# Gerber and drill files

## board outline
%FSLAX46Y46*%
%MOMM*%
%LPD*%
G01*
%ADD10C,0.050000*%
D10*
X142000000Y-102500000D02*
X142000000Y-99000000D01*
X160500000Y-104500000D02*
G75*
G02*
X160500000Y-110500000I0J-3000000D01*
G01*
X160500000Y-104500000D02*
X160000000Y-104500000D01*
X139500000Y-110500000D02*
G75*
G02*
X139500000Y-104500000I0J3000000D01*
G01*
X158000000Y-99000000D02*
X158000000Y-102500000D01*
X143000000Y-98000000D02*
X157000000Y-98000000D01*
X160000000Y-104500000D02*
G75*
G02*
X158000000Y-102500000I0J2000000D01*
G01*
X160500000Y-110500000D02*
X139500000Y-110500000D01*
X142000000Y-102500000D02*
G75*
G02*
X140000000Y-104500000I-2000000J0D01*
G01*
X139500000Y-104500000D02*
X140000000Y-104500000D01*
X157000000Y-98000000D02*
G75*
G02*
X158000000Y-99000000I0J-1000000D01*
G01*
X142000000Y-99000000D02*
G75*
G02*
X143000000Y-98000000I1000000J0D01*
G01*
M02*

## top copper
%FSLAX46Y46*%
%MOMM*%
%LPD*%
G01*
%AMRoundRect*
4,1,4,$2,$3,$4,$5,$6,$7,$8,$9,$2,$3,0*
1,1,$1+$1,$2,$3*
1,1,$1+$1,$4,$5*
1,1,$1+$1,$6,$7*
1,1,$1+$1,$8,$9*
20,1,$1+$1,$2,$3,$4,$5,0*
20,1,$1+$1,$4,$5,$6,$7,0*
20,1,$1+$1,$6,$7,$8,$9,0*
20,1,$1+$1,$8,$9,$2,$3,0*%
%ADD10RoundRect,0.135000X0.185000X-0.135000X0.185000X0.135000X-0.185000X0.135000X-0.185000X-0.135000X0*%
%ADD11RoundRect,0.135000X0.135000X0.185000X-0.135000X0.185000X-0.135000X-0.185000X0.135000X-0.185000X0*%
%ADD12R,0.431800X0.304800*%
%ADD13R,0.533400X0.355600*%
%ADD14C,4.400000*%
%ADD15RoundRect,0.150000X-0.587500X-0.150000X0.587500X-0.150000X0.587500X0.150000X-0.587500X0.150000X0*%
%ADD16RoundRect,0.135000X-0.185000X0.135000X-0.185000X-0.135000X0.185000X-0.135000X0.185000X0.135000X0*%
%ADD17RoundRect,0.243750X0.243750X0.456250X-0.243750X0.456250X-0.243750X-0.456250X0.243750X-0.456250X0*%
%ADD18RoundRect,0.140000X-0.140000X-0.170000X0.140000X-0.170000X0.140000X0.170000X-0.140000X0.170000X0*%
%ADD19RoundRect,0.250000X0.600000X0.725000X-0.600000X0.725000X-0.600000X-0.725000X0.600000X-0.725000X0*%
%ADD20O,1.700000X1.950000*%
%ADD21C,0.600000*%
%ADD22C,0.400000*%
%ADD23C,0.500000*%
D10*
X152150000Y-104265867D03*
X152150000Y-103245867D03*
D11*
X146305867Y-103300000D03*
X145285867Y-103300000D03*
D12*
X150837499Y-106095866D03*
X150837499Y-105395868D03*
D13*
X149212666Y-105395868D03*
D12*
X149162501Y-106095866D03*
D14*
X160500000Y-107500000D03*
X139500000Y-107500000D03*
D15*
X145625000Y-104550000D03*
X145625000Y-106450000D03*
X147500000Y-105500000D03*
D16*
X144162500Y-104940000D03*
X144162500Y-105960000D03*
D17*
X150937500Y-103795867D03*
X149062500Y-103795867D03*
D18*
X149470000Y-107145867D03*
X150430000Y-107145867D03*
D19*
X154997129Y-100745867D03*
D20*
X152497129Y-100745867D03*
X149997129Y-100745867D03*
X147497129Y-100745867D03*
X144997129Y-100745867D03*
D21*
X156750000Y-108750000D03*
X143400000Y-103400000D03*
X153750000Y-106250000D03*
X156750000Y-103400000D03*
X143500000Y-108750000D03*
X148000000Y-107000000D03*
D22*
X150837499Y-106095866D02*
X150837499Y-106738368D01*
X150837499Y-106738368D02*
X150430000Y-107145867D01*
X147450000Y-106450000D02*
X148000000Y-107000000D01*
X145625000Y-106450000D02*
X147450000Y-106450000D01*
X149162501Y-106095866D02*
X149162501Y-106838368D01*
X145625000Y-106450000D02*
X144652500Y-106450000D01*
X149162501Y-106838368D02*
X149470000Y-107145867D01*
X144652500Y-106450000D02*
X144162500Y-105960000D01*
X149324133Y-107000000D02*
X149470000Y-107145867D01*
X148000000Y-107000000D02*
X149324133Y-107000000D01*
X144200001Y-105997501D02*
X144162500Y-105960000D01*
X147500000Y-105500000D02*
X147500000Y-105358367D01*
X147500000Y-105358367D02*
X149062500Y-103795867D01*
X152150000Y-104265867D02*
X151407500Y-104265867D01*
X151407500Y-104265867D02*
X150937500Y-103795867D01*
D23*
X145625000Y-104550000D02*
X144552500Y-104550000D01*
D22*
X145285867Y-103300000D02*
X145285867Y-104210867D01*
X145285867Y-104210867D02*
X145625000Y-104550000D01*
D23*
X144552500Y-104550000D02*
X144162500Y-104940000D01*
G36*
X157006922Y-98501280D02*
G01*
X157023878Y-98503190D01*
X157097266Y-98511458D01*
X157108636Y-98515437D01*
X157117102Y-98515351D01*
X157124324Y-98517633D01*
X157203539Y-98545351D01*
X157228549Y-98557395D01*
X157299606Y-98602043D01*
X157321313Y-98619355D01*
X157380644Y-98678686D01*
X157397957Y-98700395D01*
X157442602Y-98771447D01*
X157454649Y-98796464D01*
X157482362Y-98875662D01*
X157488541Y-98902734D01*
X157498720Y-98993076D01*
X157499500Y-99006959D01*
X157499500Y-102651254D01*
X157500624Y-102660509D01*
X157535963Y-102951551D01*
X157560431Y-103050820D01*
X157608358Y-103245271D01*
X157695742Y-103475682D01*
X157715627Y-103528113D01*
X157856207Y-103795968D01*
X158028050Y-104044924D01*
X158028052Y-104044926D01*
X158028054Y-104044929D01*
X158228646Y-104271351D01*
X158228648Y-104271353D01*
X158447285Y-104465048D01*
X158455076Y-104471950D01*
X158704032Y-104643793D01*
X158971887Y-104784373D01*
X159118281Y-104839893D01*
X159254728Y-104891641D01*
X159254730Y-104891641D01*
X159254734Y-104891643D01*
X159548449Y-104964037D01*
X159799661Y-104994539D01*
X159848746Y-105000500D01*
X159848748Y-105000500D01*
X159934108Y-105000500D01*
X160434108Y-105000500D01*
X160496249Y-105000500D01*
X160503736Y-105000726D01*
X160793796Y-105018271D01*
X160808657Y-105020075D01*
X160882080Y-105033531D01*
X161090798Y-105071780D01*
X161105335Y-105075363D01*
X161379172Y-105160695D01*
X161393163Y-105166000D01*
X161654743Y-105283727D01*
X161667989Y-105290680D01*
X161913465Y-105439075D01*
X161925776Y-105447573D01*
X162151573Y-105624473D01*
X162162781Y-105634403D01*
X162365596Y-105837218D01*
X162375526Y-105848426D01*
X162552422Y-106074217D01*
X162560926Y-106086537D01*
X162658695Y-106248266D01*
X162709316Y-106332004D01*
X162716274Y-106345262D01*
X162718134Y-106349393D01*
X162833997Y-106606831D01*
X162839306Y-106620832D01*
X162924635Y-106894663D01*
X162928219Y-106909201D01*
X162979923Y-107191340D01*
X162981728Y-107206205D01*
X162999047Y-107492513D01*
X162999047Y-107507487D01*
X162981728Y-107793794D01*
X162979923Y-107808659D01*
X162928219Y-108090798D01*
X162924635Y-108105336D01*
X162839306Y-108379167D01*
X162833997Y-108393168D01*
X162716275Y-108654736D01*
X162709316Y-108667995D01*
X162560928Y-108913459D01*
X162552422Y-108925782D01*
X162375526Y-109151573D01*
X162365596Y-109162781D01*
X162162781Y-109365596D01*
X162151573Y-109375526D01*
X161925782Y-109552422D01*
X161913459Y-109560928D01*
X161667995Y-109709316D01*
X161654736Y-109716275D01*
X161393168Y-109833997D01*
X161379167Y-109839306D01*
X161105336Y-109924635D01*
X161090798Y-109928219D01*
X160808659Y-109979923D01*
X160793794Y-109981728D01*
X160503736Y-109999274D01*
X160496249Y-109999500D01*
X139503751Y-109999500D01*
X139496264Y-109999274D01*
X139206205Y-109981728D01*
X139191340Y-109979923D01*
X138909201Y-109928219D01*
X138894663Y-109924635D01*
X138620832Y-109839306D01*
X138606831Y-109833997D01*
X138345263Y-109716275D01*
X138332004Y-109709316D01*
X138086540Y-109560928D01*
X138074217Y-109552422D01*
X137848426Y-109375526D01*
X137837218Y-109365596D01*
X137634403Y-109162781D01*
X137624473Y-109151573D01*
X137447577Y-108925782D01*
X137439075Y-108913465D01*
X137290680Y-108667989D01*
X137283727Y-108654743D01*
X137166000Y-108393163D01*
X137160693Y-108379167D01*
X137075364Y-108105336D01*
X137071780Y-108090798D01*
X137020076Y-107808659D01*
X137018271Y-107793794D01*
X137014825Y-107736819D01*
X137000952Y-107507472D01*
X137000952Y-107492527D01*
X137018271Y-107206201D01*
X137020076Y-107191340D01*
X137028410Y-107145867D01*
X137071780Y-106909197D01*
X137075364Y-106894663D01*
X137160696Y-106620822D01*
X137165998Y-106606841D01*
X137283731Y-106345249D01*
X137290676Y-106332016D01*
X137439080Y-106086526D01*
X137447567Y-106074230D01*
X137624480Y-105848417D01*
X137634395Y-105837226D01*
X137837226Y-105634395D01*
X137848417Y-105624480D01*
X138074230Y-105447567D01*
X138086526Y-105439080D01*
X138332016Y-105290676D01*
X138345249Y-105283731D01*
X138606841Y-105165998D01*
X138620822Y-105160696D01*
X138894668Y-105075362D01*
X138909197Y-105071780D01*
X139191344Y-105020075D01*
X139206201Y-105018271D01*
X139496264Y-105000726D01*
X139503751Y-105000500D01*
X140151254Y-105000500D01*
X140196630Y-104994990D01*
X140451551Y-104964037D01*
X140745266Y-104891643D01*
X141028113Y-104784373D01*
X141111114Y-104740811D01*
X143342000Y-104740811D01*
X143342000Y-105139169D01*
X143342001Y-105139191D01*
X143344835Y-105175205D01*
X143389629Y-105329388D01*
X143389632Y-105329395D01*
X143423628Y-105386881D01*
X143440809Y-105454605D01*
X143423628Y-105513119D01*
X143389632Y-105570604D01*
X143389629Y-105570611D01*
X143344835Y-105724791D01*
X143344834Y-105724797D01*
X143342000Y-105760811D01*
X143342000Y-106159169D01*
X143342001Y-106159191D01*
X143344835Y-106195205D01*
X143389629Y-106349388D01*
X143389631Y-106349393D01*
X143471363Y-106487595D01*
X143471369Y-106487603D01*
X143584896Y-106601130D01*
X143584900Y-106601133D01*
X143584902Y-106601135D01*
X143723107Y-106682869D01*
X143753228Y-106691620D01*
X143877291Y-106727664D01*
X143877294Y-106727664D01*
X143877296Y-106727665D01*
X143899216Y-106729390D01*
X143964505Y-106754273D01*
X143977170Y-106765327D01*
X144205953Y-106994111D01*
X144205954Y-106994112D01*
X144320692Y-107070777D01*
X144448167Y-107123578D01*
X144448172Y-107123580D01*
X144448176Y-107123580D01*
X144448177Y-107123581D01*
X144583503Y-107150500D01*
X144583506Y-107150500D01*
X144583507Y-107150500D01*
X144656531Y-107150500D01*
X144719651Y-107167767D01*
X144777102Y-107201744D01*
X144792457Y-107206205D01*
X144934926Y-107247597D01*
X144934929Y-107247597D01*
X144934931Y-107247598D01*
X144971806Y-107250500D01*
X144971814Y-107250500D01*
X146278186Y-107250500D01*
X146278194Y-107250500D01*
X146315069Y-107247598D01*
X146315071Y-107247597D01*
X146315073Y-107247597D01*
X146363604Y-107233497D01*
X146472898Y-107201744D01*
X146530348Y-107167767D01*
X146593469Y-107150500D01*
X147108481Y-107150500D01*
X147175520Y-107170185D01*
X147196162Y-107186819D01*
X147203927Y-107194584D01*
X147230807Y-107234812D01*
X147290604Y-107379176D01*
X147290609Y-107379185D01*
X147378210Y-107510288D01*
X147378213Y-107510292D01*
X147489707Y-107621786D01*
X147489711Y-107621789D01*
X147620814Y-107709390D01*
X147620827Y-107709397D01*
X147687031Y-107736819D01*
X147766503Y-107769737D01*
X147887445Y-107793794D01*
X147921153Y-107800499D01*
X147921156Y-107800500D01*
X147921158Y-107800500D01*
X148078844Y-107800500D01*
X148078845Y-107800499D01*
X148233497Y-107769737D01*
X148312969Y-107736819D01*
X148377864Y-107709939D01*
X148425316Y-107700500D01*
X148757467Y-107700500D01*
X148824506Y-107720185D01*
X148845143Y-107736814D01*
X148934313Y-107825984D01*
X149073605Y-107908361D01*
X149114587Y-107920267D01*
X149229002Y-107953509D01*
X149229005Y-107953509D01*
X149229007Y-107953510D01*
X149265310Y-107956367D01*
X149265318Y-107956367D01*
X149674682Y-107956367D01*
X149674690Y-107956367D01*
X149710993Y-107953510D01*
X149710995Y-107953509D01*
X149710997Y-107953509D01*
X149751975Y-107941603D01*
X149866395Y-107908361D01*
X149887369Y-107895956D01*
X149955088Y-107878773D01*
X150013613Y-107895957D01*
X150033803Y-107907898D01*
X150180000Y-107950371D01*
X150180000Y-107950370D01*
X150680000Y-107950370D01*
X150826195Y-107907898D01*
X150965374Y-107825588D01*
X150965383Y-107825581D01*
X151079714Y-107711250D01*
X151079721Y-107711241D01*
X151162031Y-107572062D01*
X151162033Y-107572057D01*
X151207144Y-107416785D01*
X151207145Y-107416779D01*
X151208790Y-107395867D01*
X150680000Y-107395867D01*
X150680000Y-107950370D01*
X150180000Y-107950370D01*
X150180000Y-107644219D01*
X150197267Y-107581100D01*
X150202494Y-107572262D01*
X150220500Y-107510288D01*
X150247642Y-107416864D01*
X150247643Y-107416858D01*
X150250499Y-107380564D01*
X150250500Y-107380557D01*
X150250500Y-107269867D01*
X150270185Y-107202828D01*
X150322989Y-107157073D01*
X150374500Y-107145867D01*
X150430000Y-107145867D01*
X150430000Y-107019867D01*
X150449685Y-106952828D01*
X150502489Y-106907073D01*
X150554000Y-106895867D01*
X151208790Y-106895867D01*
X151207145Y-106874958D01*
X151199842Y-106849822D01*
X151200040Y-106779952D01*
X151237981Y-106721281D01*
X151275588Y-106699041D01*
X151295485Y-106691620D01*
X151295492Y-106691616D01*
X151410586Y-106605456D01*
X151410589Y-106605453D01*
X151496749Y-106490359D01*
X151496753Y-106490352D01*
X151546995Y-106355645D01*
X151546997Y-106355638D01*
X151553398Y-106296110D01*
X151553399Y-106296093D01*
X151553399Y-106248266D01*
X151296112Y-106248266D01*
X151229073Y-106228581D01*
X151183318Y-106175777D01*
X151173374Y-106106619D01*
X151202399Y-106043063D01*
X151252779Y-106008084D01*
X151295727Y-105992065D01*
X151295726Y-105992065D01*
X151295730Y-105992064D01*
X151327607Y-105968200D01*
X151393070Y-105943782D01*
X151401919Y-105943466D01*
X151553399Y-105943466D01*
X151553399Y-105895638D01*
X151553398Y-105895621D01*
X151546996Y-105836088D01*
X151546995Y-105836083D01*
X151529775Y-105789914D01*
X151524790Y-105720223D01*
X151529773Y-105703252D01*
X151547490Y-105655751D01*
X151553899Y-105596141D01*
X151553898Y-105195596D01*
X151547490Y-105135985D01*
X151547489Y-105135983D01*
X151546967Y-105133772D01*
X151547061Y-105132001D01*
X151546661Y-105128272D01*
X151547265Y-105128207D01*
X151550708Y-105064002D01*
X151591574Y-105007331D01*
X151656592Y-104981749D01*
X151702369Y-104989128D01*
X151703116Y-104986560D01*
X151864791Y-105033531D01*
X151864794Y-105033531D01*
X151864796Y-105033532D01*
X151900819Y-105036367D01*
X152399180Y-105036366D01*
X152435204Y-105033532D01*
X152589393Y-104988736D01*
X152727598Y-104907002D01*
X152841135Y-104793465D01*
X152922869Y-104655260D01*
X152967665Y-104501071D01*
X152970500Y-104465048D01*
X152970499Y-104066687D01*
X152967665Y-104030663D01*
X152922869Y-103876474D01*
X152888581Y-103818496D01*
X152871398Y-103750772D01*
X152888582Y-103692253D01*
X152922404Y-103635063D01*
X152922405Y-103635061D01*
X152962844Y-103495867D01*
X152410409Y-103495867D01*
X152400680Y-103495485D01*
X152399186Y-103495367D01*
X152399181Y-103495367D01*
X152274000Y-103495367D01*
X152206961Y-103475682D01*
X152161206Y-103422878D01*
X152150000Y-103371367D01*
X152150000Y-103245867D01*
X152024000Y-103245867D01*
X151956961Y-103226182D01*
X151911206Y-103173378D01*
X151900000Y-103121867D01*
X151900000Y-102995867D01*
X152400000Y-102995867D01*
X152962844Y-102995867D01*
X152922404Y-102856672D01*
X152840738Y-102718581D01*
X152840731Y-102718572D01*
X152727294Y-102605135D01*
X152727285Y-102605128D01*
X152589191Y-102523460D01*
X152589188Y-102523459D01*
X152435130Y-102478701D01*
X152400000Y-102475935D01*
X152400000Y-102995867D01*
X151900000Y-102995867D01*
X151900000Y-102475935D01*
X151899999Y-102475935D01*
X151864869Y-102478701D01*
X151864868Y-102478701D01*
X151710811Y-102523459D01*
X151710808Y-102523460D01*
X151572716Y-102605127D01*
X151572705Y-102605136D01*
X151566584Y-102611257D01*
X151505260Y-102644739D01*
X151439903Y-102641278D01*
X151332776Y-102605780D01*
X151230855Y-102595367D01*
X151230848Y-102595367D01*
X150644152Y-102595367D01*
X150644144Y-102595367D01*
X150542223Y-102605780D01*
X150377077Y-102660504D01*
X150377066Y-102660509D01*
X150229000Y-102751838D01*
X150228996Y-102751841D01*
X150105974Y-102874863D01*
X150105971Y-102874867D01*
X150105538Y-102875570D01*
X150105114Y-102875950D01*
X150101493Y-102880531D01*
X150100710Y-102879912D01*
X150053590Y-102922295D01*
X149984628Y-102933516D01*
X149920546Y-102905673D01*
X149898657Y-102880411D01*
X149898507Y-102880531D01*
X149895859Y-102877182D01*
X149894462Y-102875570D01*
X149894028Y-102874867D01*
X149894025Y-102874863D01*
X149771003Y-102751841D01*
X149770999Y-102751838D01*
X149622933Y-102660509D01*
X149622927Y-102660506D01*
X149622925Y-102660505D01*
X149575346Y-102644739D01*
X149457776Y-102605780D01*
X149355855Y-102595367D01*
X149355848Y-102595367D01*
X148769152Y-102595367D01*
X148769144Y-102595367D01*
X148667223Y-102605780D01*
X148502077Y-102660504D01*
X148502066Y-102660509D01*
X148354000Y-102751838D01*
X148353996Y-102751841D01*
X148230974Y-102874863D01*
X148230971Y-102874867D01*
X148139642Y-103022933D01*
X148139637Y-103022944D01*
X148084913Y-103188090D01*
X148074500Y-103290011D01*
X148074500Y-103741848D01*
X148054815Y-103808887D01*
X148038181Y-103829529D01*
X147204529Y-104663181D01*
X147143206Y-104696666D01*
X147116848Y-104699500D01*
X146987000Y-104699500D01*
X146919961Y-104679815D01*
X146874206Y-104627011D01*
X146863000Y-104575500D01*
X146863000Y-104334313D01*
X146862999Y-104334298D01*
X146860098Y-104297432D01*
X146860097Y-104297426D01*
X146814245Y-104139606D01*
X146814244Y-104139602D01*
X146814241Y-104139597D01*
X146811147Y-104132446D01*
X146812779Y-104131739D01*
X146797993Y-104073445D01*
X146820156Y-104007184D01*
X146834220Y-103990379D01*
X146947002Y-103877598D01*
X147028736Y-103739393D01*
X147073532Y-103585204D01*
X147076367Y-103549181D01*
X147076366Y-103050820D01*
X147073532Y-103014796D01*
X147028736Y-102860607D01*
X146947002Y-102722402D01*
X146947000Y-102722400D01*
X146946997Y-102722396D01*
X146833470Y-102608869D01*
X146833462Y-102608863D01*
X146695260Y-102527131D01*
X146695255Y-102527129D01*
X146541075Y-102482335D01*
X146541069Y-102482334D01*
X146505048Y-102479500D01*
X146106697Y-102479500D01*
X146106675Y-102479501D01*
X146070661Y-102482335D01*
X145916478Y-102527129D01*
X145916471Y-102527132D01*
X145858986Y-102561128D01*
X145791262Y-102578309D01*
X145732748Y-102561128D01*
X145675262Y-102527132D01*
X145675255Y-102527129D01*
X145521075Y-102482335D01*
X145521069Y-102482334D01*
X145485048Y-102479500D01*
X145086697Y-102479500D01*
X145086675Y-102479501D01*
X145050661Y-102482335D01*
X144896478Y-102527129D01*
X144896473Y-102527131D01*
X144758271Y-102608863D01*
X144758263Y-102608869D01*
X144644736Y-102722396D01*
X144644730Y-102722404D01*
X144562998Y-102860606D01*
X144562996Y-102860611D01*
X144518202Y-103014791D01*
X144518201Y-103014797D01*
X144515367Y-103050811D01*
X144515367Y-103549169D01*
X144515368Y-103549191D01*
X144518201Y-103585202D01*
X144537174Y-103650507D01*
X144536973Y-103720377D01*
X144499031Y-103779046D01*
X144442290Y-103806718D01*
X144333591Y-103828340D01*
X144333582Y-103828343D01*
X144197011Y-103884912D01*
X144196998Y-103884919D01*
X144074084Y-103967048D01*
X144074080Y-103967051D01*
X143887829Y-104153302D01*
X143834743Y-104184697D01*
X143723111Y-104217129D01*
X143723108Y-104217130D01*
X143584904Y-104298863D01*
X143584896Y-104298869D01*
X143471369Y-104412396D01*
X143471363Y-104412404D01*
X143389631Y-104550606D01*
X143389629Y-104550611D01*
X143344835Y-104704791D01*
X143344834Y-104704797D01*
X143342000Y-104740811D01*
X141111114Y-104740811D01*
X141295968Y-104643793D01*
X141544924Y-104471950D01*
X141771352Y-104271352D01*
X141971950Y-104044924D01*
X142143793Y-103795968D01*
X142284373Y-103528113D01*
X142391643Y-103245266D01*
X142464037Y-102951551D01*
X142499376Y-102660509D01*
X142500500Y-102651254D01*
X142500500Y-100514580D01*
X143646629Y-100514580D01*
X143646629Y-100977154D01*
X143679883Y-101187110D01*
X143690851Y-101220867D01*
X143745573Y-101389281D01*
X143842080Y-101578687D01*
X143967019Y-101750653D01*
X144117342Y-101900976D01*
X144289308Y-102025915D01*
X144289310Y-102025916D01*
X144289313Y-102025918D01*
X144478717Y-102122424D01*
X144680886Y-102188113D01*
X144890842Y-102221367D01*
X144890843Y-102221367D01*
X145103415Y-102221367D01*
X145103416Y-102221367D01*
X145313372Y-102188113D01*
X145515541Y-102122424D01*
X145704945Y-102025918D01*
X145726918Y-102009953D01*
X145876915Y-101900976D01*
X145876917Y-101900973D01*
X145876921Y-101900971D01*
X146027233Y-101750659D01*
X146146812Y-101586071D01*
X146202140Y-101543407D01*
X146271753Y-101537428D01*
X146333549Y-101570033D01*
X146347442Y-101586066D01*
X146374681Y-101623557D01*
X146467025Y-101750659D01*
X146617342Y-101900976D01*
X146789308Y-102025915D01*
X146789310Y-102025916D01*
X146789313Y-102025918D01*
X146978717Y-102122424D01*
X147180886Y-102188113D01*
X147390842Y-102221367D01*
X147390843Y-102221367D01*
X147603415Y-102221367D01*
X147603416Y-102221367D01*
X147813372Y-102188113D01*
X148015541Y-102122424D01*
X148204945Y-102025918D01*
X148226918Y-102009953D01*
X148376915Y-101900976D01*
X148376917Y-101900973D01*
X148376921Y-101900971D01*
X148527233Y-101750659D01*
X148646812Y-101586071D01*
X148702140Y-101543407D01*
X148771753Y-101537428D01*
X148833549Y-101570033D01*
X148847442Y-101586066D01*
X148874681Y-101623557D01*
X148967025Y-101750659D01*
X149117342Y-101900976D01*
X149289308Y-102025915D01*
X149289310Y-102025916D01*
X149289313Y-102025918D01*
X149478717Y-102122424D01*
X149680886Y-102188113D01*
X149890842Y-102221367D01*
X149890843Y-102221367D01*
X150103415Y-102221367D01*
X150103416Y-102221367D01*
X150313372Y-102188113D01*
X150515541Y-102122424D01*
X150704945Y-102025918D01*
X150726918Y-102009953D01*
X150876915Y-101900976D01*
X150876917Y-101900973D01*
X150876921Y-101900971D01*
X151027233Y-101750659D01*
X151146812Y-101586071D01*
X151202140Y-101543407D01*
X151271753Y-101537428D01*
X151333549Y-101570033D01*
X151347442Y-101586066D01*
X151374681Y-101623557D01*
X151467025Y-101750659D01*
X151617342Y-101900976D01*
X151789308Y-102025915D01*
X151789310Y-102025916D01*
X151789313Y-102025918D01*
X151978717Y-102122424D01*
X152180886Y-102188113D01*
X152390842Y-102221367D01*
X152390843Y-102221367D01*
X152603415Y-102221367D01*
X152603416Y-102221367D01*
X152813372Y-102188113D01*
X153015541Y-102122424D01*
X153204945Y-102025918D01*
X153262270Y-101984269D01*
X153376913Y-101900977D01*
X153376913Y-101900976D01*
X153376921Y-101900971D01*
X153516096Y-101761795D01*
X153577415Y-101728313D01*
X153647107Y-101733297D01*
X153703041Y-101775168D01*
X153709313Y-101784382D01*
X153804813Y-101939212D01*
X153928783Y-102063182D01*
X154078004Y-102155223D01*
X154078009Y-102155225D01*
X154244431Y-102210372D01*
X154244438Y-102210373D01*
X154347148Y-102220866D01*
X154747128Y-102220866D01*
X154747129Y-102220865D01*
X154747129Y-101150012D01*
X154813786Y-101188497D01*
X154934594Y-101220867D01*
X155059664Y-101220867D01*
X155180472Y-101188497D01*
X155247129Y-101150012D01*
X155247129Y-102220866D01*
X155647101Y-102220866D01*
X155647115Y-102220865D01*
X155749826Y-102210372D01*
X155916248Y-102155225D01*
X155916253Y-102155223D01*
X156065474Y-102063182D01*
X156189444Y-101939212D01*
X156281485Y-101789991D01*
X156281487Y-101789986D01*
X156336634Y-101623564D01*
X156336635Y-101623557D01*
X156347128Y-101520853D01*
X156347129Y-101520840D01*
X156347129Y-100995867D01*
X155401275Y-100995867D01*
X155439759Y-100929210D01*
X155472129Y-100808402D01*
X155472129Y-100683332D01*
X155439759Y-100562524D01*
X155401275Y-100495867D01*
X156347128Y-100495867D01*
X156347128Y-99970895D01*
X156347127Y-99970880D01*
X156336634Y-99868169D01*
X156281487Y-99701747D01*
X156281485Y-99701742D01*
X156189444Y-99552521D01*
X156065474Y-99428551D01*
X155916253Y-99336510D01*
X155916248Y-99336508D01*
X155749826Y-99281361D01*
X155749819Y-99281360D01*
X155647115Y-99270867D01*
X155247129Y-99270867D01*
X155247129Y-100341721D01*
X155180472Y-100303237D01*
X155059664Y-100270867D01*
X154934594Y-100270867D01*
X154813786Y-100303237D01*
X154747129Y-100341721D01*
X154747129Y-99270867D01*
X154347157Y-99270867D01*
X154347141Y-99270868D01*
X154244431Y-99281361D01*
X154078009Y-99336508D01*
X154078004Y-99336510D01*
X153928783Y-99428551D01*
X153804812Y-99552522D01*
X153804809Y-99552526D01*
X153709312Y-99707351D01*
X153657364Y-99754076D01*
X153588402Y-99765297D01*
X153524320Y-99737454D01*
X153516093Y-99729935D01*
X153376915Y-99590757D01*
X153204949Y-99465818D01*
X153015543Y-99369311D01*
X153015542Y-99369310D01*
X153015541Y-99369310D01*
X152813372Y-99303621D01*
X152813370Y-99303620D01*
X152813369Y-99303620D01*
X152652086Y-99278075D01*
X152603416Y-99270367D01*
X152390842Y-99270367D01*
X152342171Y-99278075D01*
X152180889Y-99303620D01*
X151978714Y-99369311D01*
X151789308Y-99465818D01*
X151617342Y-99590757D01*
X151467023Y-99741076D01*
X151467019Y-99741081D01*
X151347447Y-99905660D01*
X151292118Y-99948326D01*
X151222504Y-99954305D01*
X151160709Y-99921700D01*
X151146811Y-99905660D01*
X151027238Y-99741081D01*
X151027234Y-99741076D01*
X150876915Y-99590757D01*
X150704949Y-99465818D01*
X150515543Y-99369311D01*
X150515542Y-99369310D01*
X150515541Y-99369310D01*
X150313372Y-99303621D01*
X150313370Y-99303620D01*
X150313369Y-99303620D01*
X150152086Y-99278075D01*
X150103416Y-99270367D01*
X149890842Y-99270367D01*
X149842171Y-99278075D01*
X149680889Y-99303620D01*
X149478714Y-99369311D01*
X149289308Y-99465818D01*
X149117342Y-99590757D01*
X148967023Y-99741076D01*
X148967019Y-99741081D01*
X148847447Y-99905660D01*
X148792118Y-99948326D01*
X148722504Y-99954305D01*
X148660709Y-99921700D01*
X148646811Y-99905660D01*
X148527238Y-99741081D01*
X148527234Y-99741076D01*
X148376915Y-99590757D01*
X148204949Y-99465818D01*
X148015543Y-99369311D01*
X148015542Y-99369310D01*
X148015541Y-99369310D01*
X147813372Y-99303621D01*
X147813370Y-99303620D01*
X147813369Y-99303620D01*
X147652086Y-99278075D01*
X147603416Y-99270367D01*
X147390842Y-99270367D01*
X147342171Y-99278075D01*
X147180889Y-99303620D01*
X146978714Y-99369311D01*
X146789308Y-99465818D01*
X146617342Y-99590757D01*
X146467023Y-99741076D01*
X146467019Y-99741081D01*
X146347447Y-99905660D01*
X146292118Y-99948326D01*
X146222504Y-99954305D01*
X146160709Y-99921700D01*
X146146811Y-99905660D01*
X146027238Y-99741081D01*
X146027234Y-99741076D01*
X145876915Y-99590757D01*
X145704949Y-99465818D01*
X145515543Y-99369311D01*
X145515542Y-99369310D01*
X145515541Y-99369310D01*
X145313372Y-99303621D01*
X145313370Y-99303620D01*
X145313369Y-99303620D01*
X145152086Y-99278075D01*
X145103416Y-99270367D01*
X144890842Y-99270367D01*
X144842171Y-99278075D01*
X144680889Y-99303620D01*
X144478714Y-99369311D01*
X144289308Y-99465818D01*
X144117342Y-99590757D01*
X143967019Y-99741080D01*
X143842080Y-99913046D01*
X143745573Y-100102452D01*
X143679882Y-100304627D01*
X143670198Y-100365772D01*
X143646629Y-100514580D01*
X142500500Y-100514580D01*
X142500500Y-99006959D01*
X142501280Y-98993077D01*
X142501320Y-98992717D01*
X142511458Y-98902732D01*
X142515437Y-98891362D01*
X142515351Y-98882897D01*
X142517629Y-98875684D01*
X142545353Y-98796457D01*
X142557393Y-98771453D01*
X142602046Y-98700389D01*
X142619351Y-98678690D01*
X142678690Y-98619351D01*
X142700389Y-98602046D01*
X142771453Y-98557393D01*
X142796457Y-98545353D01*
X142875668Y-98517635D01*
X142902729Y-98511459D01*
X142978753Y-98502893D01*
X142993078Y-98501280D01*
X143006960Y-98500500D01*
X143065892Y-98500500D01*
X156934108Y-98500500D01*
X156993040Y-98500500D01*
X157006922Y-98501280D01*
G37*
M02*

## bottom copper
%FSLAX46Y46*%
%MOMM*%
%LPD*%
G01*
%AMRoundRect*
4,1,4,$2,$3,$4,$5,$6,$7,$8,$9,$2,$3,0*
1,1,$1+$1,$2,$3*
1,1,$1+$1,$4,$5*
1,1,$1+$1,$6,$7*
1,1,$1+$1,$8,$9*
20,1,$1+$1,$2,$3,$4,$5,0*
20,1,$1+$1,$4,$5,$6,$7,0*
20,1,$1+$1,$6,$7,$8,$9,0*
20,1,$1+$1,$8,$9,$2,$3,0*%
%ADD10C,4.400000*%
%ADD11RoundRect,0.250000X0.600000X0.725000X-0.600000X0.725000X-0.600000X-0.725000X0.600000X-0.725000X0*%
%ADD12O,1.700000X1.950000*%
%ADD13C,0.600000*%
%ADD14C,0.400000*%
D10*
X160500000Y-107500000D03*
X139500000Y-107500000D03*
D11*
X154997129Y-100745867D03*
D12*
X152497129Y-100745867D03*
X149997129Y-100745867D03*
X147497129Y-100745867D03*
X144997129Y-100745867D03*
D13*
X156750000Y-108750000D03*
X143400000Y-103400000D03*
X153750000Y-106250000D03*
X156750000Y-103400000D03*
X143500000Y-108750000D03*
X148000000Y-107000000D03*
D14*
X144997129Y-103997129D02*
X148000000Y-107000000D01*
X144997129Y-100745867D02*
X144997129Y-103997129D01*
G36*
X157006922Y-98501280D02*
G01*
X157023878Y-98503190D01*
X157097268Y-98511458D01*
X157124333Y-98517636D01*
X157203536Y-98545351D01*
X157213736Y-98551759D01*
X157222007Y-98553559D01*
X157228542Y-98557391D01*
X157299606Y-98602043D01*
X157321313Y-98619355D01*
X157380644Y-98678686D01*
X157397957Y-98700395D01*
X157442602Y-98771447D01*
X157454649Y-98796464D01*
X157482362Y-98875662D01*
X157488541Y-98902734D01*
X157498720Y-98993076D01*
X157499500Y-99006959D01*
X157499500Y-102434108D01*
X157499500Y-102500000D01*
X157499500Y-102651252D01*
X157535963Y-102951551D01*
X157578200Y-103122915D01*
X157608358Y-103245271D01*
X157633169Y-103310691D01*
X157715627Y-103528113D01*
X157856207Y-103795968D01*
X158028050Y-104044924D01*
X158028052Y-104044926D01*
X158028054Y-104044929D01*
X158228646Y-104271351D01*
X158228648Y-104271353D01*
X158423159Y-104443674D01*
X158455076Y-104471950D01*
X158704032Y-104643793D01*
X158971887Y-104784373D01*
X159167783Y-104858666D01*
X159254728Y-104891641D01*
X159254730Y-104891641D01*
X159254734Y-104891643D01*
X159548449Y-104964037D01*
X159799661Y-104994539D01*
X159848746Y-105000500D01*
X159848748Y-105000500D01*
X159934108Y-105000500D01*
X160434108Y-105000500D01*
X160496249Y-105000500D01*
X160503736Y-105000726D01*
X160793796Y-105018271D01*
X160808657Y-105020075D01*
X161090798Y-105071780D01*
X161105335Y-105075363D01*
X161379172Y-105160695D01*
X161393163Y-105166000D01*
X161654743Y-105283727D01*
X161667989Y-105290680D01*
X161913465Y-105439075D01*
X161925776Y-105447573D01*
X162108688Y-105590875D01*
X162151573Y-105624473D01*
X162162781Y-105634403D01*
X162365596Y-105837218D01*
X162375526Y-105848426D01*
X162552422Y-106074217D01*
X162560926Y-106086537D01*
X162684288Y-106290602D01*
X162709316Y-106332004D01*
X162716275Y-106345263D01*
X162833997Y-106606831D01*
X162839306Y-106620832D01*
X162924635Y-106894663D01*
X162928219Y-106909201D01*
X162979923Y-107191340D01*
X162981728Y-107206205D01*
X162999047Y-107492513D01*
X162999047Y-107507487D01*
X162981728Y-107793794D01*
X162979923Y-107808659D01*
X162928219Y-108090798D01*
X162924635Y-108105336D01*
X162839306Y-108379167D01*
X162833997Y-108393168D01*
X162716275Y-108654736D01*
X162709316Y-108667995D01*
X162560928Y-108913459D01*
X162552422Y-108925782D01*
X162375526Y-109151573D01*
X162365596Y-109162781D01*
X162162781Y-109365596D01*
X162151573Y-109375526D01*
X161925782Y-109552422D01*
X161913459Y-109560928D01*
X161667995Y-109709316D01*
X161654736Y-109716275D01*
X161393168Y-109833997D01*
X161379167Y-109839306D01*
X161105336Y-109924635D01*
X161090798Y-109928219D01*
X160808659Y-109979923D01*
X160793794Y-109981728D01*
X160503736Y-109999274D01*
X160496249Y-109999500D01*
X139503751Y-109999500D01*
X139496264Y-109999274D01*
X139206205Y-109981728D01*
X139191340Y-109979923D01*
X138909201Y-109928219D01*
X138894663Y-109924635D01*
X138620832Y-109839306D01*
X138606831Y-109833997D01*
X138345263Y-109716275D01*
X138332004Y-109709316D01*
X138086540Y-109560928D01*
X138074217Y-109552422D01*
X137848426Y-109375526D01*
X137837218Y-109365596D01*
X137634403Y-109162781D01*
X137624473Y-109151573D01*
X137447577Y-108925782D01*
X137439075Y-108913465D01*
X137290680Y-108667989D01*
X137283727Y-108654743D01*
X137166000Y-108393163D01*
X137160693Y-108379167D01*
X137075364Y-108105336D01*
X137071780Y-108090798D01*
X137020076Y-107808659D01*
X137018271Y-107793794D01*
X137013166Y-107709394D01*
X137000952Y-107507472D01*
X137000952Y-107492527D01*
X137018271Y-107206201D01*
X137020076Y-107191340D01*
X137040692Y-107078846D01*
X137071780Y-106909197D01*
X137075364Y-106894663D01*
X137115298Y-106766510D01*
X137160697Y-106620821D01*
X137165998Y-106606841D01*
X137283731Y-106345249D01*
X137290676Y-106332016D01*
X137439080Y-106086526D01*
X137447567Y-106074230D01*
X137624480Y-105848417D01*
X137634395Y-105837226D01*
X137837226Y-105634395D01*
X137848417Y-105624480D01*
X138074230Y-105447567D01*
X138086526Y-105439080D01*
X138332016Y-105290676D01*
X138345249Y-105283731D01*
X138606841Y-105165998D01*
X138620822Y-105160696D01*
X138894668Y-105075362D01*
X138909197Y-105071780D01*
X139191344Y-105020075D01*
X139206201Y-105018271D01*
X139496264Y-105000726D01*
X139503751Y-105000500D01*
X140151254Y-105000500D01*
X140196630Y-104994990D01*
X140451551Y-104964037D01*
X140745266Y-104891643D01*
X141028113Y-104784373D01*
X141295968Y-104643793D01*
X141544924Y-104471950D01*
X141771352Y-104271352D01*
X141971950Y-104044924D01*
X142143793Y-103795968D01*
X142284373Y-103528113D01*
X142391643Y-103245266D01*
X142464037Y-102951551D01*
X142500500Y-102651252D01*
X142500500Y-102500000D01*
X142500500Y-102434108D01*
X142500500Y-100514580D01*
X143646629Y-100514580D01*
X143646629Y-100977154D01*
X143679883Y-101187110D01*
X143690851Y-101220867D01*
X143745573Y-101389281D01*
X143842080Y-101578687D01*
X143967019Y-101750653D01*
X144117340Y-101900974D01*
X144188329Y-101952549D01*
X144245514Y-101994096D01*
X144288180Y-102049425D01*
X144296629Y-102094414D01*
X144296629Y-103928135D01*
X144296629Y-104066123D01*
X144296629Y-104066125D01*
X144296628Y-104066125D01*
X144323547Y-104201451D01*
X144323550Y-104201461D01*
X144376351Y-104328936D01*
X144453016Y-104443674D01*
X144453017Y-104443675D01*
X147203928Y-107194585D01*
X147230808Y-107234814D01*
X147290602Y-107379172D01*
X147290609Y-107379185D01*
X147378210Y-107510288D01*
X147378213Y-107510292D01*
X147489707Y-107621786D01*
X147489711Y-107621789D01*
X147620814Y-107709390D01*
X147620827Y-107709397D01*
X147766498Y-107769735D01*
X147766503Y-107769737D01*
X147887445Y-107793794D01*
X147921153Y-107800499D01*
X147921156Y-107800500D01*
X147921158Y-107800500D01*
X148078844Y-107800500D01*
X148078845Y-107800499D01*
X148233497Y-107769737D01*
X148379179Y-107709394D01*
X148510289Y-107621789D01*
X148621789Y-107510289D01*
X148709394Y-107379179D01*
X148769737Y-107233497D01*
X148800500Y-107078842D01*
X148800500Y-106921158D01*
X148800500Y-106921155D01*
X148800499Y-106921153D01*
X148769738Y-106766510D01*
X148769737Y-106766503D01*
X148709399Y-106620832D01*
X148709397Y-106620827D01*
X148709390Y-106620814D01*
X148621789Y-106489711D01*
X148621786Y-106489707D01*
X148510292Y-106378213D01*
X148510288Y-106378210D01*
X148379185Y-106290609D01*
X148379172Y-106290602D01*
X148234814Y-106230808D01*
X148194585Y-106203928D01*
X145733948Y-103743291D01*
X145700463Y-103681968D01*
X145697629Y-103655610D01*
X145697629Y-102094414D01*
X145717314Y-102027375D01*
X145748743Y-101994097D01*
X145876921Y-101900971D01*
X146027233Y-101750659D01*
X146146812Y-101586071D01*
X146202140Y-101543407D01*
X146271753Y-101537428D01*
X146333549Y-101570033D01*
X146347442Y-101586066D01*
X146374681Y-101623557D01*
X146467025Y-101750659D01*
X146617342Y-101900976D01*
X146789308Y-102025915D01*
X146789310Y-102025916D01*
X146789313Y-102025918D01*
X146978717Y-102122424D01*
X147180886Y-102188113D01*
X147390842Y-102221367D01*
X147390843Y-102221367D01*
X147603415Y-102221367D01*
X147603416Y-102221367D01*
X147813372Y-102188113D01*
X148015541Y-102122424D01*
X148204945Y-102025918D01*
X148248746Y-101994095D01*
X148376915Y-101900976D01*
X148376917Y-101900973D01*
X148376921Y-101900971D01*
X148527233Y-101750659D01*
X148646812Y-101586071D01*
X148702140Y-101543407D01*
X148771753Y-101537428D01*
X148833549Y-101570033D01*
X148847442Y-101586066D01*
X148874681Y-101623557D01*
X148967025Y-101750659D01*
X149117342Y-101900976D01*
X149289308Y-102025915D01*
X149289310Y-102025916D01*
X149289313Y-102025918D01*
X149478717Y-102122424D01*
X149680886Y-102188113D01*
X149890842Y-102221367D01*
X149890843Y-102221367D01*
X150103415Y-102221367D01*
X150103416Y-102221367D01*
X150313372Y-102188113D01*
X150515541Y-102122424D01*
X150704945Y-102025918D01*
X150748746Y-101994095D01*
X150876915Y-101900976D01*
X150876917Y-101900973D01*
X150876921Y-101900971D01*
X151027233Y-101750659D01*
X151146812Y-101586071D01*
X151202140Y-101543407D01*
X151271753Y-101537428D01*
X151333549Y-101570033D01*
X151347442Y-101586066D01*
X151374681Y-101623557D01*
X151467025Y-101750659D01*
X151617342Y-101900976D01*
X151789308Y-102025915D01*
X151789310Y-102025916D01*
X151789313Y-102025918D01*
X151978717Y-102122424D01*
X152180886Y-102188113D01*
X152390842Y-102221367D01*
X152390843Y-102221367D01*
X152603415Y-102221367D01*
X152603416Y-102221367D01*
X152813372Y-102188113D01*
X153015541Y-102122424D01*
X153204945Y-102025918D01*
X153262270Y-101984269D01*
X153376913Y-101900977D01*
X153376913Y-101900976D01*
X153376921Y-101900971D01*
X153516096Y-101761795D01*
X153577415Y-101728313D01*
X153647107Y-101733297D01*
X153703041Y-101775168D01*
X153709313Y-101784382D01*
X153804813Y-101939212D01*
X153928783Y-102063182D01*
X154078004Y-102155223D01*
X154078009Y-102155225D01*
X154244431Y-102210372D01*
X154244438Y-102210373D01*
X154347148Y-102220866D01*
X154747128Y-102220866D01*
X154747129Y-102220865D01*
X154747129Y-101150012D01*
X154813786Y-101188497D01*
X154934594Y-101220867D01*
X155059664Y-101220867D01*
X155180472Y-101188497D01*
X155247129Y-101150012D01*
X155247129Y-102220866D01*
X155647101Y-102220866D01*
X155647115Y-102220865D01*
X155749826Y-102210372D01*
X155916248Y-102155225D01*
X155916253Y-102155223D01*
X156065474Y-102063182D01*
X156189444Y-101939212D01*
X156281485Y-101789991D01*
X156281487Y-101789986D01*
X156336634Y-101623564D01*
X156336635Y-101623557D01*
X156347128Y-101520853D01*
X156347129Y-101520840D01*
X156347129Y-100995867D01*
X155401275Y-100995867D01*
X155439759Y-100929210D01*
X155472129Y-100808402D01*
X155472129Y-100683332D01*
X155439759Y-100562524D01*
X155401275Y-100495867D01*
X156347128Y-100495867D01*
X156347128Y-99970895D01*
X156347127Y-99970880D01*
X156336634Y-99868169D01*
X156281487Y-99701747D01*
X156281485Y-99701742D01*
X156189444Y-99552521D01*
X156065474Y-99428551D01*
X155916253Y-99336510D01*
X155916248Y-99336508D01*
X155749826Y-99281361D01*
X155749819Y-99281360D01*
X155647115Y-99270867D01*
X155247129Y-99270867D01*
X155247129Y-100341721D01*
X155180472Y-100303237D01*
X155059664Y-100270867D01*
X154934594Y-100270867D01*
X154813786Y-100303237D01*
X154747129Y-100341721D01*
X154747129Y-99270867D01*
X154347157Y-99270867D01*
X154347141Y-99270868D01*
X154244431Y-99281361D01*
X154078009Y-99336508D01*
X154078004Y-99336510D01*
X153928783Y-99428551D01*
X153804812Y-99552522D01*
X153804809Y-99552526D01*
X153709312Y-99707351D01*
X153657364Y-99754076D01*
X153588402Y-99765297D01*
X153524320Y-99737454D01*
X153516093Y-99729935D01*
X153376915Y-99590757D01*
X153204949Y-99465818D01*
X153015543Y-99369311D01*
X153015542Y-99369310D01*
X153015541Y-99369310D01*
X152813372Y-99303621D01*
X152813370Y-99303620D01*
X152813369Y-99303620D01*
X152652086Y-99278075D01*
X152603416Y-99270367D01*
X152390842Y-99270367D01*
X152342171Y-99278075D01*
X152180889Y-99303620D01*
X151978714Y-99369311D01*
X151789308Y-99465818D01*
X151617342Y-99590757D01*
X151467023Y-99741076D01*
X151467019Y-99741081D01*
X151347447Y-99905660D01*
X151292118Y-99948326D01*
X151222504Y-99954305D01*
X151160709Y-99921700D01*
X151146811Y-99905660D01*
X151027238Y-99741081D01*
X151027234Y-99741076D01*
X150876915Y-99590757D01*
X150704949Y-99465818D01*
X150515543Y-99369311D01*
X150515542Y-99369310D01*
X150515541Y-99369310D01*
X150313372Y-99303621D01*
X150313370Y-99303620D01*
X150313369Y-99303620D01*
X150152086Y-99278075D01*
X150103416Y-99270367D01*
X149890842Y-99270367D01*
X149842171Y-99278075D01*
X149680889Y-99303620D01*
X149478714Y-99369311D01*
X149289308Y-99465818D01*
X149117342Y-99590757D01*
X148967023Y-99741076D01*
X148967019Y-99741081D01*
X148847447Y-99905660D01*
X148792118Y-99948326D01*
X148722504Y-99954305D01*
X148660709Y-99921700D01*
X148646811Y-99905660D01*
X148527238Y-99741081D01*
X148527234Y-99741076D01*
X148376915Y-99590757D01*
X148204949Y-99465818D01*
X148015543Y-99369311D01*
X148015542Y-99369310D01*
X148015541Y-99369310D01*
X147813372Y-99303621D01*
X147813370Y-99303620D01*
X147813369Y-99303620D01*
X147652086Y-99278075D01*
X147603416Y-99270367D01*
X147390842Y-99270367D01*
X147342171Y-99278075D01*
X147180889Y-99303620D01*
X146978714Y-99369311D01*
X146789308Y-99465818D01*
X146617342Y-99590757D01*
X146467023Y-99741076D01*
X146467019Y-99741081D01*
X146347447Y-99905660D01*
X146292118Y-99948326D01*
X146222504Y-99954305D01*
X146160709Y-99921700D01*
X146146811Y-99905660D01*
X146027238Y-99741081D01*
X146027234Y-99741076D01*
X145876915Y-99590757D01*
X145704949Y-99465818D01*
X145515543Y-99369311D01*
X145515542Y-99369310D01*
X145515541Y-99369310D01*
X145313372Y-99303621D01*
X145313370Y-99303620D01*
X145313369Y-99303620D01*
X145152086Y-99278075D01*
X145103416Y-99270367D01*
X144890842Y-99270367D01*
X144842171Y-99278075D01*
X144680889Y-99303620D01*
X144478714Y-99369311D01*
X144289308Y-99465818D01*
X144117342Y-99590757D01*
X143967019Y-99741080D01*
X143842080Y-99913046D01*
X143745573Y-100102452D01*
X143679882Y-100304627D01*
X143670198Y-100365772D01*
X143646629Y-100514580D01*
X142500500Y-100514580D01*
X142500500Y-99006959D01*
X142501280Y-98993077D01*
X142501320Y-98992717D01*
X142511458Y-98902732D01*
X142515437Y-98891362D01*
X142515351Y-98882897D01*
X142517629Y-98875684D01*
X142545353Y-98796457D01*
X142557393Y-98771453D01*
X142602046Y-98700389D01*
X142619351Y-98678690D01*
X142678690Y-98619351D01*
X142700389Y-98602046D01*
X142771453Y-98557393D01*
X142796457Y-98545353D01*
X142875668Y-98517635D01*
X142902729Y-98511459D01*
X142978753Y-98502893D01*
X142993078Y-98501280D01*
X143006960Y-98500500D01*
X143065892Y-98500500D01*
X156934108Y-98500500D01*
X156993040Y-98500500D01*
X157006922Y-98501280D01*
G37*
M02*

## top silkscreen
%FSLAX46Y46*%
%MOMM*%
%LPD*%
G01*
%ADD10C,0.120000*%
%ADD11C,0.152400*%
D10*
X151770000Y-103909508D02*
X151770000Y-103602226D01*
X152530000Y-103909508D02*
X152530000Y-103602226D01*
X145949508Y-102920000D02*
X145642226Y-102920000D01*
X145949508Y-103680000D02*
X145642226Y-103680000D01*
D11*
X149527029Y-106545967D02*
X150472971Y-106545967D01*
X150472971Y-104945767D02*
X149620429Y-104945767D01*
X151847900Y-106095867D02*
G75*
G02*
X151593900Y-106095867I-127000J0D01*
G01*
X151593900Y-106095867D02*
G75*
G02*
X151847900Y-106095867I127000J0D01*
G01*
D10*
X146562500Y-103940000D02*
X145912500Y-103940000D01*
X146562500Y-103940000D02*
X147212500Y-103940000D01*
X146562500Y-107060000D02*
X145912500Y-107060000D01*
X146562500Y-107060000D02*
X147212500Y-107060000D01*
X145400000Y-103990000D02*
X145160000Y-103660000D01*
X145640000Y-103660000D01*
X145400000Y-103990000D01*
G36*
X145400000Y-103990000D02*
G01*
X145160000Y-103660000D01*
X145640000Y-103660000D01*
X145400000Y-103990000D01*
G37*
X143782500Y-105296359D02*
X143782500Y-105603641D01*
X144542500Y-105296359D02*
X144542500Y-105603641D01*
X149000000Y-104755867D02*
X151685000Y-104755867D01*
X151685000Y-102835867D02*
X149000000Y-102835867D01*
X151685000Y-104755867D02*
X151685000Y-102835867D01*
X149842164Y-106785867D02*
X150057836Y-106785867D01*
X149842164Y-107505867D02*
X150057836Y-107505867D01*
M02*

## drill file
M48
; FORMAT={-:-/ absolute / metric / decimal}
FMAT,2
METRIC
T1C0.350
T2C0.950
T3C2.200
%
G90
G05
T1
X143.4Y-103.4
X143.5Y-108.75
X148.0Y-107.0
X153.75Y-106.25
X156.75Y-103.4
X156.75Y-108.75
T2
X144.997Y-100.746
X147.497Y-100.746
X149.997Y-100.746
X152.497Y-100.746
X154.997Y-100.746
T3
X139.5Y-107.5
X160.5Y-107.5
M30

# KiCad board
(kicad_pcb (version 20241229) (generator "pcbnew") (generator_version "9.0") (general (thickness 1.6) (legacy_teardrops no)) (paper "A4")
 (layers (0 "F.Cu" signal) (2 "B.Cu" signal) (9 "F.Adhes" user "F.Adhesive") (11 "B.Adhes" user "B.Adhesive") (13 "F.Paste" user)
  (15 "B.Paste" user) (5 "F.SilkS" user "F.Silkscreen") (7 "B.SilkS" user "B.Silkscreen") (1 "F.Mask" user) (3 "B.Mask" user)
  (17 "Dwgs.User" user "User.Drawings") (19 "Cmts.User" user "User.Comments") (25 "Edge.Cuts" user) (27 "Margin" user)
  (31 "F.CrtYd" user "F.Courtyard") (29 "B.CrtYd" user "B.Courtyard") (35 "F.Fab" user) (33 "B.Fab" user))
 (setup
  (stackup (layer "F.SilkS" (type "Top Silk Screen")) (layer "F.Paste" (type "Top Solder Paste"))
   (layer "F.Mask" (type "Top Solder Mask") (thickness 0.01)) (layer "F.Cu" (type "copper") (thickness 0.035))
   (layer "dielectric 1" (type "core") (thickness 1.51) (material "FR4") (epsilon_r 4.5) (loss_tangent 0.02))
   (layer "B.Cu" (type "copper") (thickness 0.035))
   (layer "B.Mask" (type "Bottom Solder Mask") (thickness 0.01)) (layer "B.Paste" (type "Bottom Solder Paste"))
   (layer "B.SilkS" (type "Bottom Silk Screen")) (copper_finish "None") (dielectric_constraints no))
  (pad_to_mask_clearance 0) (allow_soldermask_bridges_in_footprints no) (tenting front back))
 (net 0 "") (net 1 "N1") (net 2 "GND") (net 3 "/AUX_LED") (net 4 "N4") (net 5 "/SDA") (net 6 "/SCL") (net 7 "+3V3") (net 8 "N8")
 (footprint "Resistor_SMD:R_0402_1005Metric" (layer "F.Cu") (at 152.15 103.755867 90)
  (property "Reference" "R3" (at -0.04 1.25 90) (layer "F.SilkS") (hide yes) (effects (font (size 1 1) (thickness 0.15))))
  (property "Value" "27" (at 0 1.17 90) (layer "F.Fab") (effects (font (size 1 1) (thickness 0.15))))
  (fp_line (start -0.153641 -0.38) (end 0.153641 -0.38) (stroke (width 0.12) (type solid)) (layer "F.SilkS"))
  (fp_line (start -0.153641 0.38) (end 0.153641 0.38) (stroke (width 0.12) (type solid)) (layer "F.SilkS"))
  (pad "1" smd roundrect (at -0.51 0 90) (size 0.54 0.64) (layers "F.Cu" "F.Mask" "F.Paste") (roundrect_rratio 0.25) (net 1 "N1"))
  (pad "2" smd roundrect (at 0.51 0 90) (size 0.54 0.64) (layers "F.Cu" "F.Mask" "F.Paste") (roundrect_rratio 0.25) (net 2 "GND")))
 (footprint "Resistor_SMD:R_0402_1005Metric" (layer "F.Cu") (at 145.795867 103.3 180)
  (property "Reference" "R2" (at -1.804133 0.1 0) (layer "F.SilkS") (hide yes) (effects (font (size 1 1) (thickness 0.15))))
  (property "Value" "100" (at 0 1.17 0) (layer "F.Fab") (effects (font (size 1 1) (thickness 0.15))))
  (fp_line (start -0.153641 0.38) (end 0.153641 0.38) (stroke (width 0.12) (type solid)) (layer "F.SilkS"))
  (fp_line (start -0.153641 -0.38) (end 0.153641 -0.38) (stroke (width 0.12) (type solid)) (layer "F.SilkS"))
  (pad "1" smd roundrect (at -0.51 0 180) (size 0.54 0.64) (layers "F.Cu" "F.Mask" "F.Paste") (roundrect_rratio 0.25) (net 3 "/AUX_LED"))
  (pad "2" smd roundrect (at 0.51 0 180) (size 0.54 0.64) (layers "F.Cu" "F.Mask" "F.Paste") (roundrect_rratio 0.25) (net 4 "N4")))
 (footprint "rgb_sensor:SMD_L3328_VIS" (layer "F.Cu") (at 150 105.745867 180)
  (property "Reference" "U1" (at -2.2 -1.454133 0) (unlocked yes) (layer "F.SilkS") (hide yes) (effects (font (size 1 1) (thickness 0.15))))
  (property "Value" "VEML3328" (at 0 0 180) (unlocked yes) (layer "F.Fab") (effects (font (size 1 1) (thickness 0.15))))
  (fp_line (start 0.472971 -0.8001) (end -0.472971 -0.8001) (stroke (width 0.1524) (type solid)) (layer "F.SilkS"))
  (fp_line (start -0.472971 0.8001) (end 0.379571 0.8001) (stroke (width 0.1524) (type solid)) (layer "F.SilkS"))
  (fp_circle (center -1.7209 -0.35) (end -1.5939 -0.35) (stroke (width 0.1524) (type solid)) (fill no) (layer "F.SilkS"))
  (pad "1" smd rect (at -0.837499 -0.349999 180) (size 0.4318 0.3048) (layers "F.Cu" "F.Mask" "F.Paste") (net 2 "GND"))
  (pad "2" smd rect (at -0.837499 0.349999 180) (size 0.4318 0.3048) (layers "F.Cu" "F.Mask" "F.Paste") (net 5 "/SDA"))
  (pad "3" smd rect (at 0.787334 0.349999 180) (size 0.5334 0.3556) (layers "F.Cu" "F.Mask" "F.Paste") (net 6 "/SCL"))
  (pad "4" smd rect (at 0.837499 -0.349999 180) (size 0.4318 0.3048) (layers "F.Cu" "F.Mask" "F.Paste") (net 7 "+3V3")))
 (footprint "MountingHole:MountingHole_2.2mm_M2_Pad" (layer "F.Cu") (at 160.5 107.5)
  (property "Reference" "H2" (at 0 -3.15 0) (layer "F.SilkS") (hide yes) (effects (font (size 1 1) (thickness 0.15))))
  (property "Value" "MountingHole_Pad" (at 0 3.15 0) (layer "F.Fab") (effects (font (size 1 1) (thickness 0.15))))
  (pad "1" thru_hole circle (at 0 0) (size 4.4 4.4) (drill 2.2) (layers "*.Cu" "*.Mask") (remove_unused_layers no) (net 2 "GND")
   (zone_connect 2)))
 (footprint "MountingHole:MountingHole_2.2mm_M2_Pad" (layer "F.Cu") (at 139.5 107.5)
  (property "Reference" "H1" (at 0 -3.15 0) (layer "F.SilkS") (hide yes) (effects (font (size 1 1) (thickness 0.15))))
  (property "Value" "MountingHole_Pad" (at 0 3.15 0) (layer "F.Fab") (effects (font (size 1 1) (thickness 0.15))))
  (pad "1" thru_hole circle (at 0 0) (size 4.4 4.4) (drill 2.2) (layers "*.Cu" "*.Mask") (remove_unused_layers no) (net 2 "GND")
   (zone_connect 2)))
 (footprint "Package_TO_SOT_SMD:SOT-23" (layer "F.Cu") (at 146.5625 105.5)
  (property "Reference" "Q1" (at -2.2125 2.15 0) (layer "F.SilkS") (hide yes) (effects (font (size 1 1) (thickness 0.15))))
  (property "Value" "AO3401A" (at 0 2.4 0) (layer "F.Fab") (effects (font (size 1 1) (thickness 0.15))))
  (fp_line (start 0 -1.56) (end -0.65 -1.56) (stroke (width 0.12) (type solid)) (layer "F.SilkS"))
  (fp_line (start 0 -1.56) (end 0.65 -1.56) (stroke (width 0.12) (type solid)) (layer "F.SilkS"))
  (fp_line (start 0 1.56) (end -0.65 1.56) (stroke (width 0.12) (type solid)) (layer "F.SilkS"))
  (fp_line (start 0 1.56) (end 0.65 1.56) (stroke (width 0.12) (type solid)) (layer "F.SilkS"))
  (fp_poly (pts (xy -1.1625 -1.51) (xy -1.4025 -1.84) (xy -0.9225 -1.84)) (stroke (width 0.12) (type solid)) (fill yes) (layer "F.SilkS"))
  (pad "1" smd roundrect (at -0.9375 -0.95) (size 1.475 0.6) (layers "F.Cu" "F.Mask" "F.Paste") (roundrect_rratio 0.25) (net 4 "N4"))
  (pad "2" smd roundrect (at -0.9375 0.95) (size 1.475 0.6) (layers "F.Cu" "F.Mask" "F.Paste") (roundrect_rratio 0.25) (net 7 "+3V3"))
  (pad "3" smd roundrect (at 0.9375 0) (size 1.475 0.6) (layers "F.Cu" "F.Mask" "F.Paste") (roundrect_rratio 0.25) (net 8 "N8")))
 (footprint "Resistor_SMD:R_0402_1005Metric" (layer "F.Cu") (at 144.1625 105.45 -90)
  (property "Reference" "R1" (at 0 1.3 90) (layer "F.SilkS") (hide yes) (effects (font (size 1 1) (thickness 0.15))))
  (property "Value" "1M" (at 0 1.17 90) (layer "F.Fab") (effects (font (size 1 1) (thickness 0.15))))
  (fp_line (start -0.153641 0.38) (end 0.153641 0.38) (stroke (width 0.12) (type solid)) (layer "F.SilkS"))
  (fp_line (start -0.153641 -0.38) (end 0.153641 -0.38) (stroke (width 0.12) (type solid)) (layer "F.SilkS"))
  (pad "1" smd roundrect (at -0.51 0 270) (size 0.54 0.64) (layers "F.Cu" "F.Mask" "F.Paste") (roundrect_rratio 0.25) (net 4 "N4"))
  (pad "2" smd roundrect (at 0.51 0 270) (size 0.54 0.64) (layers "F.Cu" "F.Mask" "F.Paste") (roundrect_rratio 0.25) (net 7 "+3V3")))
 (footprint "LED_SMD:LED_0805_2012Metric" (layer "F.Cu") (at 150 103.795867 180)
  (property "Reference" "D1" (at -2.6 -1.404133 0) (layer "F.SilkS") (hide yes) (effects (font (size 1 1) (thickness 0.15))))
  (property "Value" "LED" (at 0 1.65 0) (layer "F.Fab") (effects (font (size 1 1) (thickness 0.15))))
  (fp_line (start 1 -0.96) (end -1.685 -0.96) (stroke (width 0.12) (type solid)) (layer "F.SilkS"))
  (fp_line (start -1.685 0.96) (end 1 0.96) (stroke (width 0.12) (type solid)) (layer "F.SilkS"))
  (fp_line (start -1.685 -0.96) (end -1.685 0.96) (stroke (width 0.12) (type solid)) (layer "F.SilkS"))
  (pad "1" smd roundrect (at -0.9375 0 180) (size 0.975 1.4) (layers "F.Cu" "F.Mask" "F.Paste") (roundrect_rratio 0.25) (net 1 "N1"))
  (pad "2" smd roundrect (at 0.9375 0 180) (size 0.975 1.4) (layers "F.Cu" "F.Mask" "F.Paste") (roundrect_rratio 0.25) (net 8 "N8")))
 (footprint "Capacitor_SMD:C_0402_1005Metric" (layer "F.Cu") (at 149.95 107.145867)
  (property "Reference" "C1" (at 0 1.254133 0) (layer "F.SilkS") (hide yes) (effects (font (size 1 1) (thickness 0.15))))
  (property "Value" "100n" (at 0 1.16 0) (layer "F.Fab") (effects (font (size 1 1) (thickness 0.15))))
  (fp_line (start -0.107836 -0.36) (end 0.107836 -0.36) (stroke (width 0.12) (type solid)) (layer "F.SilkS"))
  (fp_line (start -0.107836 0.36) (end 0.107836 0.36) (stroke (width 0.12) (type solid)) (layer "F.SilkS"))
  (pad "1" smd roundrect (at -0.48 0) (size 0.56 0.62) (layers "F.Cu" "F.Mask" "F.Paste") (roundrect_rratio 0.25) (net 7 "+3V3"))
  (pad "2" smd roundrect (at 0.48 0) (size 0.56 0.62) (layers "F.Cu" "F.Mask" "F.Paste") (roundrect_rratio 0.25) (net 2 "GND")))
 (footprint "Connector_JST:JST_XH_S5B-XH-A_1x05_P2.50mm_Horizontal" (layer "B.Cu") (at 154.997129 100.745867 180)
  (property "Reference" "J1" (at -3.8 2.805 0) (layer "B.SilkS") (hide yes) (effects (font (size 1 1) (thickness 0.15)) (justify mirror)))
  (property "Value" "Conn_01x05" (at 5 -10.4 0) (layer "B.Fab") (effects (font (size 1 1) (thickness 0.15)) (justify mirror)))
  (pad "1" thru_hole roundrect (at 0 0 180) (size 1.7 1.95) (drill 0.95) (layers "*.Cu" "*.Mask") (remove_unused_layers no)
   (roundrect_rratio 0.147059) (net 2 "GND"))
  (pad "2" thru_hole oval (at 2.5 0 180) (size 1.7 1.95) (drill 0.95) (layers "*.Cu" "*.Mask") (remove_unused_layers no) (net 5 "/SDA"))
  (pad "3" thru_hole oval (at 5 0 180) (size 1.7 1.95) (drill 0.95) (layers "*.Cu" "*.Mask") (remove_unused_layers no) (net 6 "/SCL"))
  (pad "4" thru_hole oval (at 7.5 0 180) (size 1.7 1.95) (drill 0.95) (layers "*.Cu" "*.Mask") (remove_unused_layers no) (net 3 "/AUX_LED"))
  (pad "5" thru_hole oval (at 10 0 180) (size 1.7 1.95) (drill 0.95) (layers "*.Cu" "*.Mask") (remove_unused_layers no) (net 7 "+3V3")))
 (gr_line (start 142 102.5) (end 142 99) (stroke (width 0.05) (type default)) (layer "Edge.Cuts"))
 (gr_arc (start 160.5 104.5) (mid 163.5 107.5) (end 160.5 110.5) (stroke (width 0.05) (type default)) (layer "Edge.Cuts"))
 (gr_line (start 160.5 104.5) (end 160 104.5) (stroke (width 0.05) (type default)) (layer "Edge.Cuts"))
 (gr_arc (start 139.5 110.5) (mid 136.5 107.5) (end 139.5 104.5) (stroke (width 0.05) (type default)) (layer "Edge.Cuts"))
 (gr_line (start 158 99) (end 158 102.5) (stroke (width 0.05) (type default)) (layer "Edge.Cuts"))
 (gr_line (start 143 98) (end 157 98) (stroke (width 0.05) (type default)) (layer "Edge.Cuts"))
 (gr_arc (start 160 104.5) (mid 158.585786 103.914214) (end 158 102.5) (stroke (width 0.05) (type default)) (layer "Edge.Cuts"))
 (gr_line (start 160.5 110.5) (end 139.5 110.5) (stroke (width 0.05) (type default)) (layer "Edge.Cuts"))
 (gr_arc (start 142 102.5) (mid 141.414214 103.914214) (end 140 104.5) (stroke (width 0.05) (type default)) (layer "Edge.Cuts"))
 (gr_line (start 139.5 104.5) (end 140 104.5) (stroke (width 0.05) (type default)) (layer "Edge.Cuts"))
 (gr_arc (start 157 98) (mid 157.707107 98.292893) (end 158 99) (stroke (width 0.05) (type default)) (layer "Edge.Cuts"))
 (gr_arc (start 142 99) (mid 142.292893 98.292893) (end 143 98) (stroke (width 0.05) (type default)) (layer "Edge.Cuts"))
 (segment (start 150.837499 106.095866) (end 150.837499 106.738368) (width 0.4) (layer "F.Cu") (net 2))
 (segment (start 150.837499 106.738368) (end 150.43 107.145867) (width 0.4) (layer "F.Cu") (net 2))
 (via (at 156.75 108.75) (size 0.6) (drill 0.35) (layers "F.Cu" "B.Cu") (free yes) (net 2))
 (via (at 143.4 103.4) (size 0.6) (drill 0.35) (layers "F.Cu" "B.Cu") (free yes) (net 2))
 (via (at 153.75 106.25) (size 0.6) (drill 0.35) (layers "F.Cu" "B.Cu") (free yes) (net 2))
 (via (at 156.75 103.4) (size 0.6) (drill 0.35) (layers "F.Cu" "B.Cu") (free yes) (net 2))
 (via (at 143.5 108.75) (size 0.6) (drill 0.35) (layers "F.Cu" "B.Cu") (free yes) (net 2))
 (segment (start 147.45 106.45) (end 148 107) (width 0.4) (layer "F.Cu") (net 7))
 (segment (start 145.625 106.45) (end 147.45 106.45) (width 0.4) (layer "F.Cu") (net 7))
 (segment (start 149.162501 106.095866) (end 149.162501 106.838368) (width 0.4) (layer "F.Cu") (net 7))
 (segment (start 145.625 106.45) (end 144.6525 106.45) (width 0.4) (layer "F.Cu") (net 7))
 (segment (start 149.162501 106.838368) (end 149.47 107.145867) (width 0.4) (layer "F.Cu") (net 7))
 (segment (start 144.6525 106.45) (end 144.1625 105.96) (width 0.4) (layer "F.Cu") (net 7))
 (segment (start 149.324133 107) (end 149.47 107.145867) (width 0.4) (layer "F.Cu") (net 7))
 (segment (start 148 107) (end 149.324133 107) (width 0.4) (layer "F.Cu") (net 7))
 (segment (start 144.200001 105.997501) (end 144.1625 105.96) (width 0.4) (layer "F.Cu") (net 7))
 (via (at 148 107) (size 0.6) (drill 0.35) (layers "F.Cu" "B.Cu") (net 7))
 (segment (start 144.997129 103.997129) (end 148 107) (width 0.4) (layer "B.Cu") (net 7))
 (segment (start 144.997129 100.745867) (end 144.997129 103.997129) (width 0.4) (layer "B.Cu") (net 7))
 (segment (start 147.5 105.5) (end 147.5 105.358367) (width 0.4) (layer "F.Cu") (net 8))
 (segment (start 147.5 105.358367) (end 149.0625 103.795867) (width 0.4) (layer "F.Cu") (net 8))
 (segment (start 152.15 104.265867) (end 151.4075 104.265867) (width 0.4) (layer "F.Cu") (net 1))
 (segment (start 151.4075 104.265867) (end 150.9375 103.795867) (width 0.4) (layer "F.Cu") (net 1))
 (segment (start 145.625 104.55) (end 144.5525 104.55) (width 0.5) (layer "F.Cu") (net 4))
 (segment (start 145.285867 103.3) (end 145.285867 104.210867) (width 0.4) (layer "F.Cu") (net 4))
 (segment (start 145.285867 104.210867) (end 145.625 104.55) (width 0.4) (layer "F.Cu") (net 4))
 (segment (start 144.5525 104.55) (end 144.1625 104.94) (width 0.5) (layer "F.Cu") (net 4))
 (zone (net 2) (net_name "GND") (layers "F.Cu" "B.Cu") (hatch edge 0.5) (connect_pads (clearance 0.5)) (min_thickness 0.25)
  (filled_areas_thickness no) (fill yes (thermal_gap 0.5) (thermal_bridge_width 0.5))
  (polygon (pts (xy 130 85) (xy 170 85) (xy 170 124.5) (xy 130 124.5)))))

